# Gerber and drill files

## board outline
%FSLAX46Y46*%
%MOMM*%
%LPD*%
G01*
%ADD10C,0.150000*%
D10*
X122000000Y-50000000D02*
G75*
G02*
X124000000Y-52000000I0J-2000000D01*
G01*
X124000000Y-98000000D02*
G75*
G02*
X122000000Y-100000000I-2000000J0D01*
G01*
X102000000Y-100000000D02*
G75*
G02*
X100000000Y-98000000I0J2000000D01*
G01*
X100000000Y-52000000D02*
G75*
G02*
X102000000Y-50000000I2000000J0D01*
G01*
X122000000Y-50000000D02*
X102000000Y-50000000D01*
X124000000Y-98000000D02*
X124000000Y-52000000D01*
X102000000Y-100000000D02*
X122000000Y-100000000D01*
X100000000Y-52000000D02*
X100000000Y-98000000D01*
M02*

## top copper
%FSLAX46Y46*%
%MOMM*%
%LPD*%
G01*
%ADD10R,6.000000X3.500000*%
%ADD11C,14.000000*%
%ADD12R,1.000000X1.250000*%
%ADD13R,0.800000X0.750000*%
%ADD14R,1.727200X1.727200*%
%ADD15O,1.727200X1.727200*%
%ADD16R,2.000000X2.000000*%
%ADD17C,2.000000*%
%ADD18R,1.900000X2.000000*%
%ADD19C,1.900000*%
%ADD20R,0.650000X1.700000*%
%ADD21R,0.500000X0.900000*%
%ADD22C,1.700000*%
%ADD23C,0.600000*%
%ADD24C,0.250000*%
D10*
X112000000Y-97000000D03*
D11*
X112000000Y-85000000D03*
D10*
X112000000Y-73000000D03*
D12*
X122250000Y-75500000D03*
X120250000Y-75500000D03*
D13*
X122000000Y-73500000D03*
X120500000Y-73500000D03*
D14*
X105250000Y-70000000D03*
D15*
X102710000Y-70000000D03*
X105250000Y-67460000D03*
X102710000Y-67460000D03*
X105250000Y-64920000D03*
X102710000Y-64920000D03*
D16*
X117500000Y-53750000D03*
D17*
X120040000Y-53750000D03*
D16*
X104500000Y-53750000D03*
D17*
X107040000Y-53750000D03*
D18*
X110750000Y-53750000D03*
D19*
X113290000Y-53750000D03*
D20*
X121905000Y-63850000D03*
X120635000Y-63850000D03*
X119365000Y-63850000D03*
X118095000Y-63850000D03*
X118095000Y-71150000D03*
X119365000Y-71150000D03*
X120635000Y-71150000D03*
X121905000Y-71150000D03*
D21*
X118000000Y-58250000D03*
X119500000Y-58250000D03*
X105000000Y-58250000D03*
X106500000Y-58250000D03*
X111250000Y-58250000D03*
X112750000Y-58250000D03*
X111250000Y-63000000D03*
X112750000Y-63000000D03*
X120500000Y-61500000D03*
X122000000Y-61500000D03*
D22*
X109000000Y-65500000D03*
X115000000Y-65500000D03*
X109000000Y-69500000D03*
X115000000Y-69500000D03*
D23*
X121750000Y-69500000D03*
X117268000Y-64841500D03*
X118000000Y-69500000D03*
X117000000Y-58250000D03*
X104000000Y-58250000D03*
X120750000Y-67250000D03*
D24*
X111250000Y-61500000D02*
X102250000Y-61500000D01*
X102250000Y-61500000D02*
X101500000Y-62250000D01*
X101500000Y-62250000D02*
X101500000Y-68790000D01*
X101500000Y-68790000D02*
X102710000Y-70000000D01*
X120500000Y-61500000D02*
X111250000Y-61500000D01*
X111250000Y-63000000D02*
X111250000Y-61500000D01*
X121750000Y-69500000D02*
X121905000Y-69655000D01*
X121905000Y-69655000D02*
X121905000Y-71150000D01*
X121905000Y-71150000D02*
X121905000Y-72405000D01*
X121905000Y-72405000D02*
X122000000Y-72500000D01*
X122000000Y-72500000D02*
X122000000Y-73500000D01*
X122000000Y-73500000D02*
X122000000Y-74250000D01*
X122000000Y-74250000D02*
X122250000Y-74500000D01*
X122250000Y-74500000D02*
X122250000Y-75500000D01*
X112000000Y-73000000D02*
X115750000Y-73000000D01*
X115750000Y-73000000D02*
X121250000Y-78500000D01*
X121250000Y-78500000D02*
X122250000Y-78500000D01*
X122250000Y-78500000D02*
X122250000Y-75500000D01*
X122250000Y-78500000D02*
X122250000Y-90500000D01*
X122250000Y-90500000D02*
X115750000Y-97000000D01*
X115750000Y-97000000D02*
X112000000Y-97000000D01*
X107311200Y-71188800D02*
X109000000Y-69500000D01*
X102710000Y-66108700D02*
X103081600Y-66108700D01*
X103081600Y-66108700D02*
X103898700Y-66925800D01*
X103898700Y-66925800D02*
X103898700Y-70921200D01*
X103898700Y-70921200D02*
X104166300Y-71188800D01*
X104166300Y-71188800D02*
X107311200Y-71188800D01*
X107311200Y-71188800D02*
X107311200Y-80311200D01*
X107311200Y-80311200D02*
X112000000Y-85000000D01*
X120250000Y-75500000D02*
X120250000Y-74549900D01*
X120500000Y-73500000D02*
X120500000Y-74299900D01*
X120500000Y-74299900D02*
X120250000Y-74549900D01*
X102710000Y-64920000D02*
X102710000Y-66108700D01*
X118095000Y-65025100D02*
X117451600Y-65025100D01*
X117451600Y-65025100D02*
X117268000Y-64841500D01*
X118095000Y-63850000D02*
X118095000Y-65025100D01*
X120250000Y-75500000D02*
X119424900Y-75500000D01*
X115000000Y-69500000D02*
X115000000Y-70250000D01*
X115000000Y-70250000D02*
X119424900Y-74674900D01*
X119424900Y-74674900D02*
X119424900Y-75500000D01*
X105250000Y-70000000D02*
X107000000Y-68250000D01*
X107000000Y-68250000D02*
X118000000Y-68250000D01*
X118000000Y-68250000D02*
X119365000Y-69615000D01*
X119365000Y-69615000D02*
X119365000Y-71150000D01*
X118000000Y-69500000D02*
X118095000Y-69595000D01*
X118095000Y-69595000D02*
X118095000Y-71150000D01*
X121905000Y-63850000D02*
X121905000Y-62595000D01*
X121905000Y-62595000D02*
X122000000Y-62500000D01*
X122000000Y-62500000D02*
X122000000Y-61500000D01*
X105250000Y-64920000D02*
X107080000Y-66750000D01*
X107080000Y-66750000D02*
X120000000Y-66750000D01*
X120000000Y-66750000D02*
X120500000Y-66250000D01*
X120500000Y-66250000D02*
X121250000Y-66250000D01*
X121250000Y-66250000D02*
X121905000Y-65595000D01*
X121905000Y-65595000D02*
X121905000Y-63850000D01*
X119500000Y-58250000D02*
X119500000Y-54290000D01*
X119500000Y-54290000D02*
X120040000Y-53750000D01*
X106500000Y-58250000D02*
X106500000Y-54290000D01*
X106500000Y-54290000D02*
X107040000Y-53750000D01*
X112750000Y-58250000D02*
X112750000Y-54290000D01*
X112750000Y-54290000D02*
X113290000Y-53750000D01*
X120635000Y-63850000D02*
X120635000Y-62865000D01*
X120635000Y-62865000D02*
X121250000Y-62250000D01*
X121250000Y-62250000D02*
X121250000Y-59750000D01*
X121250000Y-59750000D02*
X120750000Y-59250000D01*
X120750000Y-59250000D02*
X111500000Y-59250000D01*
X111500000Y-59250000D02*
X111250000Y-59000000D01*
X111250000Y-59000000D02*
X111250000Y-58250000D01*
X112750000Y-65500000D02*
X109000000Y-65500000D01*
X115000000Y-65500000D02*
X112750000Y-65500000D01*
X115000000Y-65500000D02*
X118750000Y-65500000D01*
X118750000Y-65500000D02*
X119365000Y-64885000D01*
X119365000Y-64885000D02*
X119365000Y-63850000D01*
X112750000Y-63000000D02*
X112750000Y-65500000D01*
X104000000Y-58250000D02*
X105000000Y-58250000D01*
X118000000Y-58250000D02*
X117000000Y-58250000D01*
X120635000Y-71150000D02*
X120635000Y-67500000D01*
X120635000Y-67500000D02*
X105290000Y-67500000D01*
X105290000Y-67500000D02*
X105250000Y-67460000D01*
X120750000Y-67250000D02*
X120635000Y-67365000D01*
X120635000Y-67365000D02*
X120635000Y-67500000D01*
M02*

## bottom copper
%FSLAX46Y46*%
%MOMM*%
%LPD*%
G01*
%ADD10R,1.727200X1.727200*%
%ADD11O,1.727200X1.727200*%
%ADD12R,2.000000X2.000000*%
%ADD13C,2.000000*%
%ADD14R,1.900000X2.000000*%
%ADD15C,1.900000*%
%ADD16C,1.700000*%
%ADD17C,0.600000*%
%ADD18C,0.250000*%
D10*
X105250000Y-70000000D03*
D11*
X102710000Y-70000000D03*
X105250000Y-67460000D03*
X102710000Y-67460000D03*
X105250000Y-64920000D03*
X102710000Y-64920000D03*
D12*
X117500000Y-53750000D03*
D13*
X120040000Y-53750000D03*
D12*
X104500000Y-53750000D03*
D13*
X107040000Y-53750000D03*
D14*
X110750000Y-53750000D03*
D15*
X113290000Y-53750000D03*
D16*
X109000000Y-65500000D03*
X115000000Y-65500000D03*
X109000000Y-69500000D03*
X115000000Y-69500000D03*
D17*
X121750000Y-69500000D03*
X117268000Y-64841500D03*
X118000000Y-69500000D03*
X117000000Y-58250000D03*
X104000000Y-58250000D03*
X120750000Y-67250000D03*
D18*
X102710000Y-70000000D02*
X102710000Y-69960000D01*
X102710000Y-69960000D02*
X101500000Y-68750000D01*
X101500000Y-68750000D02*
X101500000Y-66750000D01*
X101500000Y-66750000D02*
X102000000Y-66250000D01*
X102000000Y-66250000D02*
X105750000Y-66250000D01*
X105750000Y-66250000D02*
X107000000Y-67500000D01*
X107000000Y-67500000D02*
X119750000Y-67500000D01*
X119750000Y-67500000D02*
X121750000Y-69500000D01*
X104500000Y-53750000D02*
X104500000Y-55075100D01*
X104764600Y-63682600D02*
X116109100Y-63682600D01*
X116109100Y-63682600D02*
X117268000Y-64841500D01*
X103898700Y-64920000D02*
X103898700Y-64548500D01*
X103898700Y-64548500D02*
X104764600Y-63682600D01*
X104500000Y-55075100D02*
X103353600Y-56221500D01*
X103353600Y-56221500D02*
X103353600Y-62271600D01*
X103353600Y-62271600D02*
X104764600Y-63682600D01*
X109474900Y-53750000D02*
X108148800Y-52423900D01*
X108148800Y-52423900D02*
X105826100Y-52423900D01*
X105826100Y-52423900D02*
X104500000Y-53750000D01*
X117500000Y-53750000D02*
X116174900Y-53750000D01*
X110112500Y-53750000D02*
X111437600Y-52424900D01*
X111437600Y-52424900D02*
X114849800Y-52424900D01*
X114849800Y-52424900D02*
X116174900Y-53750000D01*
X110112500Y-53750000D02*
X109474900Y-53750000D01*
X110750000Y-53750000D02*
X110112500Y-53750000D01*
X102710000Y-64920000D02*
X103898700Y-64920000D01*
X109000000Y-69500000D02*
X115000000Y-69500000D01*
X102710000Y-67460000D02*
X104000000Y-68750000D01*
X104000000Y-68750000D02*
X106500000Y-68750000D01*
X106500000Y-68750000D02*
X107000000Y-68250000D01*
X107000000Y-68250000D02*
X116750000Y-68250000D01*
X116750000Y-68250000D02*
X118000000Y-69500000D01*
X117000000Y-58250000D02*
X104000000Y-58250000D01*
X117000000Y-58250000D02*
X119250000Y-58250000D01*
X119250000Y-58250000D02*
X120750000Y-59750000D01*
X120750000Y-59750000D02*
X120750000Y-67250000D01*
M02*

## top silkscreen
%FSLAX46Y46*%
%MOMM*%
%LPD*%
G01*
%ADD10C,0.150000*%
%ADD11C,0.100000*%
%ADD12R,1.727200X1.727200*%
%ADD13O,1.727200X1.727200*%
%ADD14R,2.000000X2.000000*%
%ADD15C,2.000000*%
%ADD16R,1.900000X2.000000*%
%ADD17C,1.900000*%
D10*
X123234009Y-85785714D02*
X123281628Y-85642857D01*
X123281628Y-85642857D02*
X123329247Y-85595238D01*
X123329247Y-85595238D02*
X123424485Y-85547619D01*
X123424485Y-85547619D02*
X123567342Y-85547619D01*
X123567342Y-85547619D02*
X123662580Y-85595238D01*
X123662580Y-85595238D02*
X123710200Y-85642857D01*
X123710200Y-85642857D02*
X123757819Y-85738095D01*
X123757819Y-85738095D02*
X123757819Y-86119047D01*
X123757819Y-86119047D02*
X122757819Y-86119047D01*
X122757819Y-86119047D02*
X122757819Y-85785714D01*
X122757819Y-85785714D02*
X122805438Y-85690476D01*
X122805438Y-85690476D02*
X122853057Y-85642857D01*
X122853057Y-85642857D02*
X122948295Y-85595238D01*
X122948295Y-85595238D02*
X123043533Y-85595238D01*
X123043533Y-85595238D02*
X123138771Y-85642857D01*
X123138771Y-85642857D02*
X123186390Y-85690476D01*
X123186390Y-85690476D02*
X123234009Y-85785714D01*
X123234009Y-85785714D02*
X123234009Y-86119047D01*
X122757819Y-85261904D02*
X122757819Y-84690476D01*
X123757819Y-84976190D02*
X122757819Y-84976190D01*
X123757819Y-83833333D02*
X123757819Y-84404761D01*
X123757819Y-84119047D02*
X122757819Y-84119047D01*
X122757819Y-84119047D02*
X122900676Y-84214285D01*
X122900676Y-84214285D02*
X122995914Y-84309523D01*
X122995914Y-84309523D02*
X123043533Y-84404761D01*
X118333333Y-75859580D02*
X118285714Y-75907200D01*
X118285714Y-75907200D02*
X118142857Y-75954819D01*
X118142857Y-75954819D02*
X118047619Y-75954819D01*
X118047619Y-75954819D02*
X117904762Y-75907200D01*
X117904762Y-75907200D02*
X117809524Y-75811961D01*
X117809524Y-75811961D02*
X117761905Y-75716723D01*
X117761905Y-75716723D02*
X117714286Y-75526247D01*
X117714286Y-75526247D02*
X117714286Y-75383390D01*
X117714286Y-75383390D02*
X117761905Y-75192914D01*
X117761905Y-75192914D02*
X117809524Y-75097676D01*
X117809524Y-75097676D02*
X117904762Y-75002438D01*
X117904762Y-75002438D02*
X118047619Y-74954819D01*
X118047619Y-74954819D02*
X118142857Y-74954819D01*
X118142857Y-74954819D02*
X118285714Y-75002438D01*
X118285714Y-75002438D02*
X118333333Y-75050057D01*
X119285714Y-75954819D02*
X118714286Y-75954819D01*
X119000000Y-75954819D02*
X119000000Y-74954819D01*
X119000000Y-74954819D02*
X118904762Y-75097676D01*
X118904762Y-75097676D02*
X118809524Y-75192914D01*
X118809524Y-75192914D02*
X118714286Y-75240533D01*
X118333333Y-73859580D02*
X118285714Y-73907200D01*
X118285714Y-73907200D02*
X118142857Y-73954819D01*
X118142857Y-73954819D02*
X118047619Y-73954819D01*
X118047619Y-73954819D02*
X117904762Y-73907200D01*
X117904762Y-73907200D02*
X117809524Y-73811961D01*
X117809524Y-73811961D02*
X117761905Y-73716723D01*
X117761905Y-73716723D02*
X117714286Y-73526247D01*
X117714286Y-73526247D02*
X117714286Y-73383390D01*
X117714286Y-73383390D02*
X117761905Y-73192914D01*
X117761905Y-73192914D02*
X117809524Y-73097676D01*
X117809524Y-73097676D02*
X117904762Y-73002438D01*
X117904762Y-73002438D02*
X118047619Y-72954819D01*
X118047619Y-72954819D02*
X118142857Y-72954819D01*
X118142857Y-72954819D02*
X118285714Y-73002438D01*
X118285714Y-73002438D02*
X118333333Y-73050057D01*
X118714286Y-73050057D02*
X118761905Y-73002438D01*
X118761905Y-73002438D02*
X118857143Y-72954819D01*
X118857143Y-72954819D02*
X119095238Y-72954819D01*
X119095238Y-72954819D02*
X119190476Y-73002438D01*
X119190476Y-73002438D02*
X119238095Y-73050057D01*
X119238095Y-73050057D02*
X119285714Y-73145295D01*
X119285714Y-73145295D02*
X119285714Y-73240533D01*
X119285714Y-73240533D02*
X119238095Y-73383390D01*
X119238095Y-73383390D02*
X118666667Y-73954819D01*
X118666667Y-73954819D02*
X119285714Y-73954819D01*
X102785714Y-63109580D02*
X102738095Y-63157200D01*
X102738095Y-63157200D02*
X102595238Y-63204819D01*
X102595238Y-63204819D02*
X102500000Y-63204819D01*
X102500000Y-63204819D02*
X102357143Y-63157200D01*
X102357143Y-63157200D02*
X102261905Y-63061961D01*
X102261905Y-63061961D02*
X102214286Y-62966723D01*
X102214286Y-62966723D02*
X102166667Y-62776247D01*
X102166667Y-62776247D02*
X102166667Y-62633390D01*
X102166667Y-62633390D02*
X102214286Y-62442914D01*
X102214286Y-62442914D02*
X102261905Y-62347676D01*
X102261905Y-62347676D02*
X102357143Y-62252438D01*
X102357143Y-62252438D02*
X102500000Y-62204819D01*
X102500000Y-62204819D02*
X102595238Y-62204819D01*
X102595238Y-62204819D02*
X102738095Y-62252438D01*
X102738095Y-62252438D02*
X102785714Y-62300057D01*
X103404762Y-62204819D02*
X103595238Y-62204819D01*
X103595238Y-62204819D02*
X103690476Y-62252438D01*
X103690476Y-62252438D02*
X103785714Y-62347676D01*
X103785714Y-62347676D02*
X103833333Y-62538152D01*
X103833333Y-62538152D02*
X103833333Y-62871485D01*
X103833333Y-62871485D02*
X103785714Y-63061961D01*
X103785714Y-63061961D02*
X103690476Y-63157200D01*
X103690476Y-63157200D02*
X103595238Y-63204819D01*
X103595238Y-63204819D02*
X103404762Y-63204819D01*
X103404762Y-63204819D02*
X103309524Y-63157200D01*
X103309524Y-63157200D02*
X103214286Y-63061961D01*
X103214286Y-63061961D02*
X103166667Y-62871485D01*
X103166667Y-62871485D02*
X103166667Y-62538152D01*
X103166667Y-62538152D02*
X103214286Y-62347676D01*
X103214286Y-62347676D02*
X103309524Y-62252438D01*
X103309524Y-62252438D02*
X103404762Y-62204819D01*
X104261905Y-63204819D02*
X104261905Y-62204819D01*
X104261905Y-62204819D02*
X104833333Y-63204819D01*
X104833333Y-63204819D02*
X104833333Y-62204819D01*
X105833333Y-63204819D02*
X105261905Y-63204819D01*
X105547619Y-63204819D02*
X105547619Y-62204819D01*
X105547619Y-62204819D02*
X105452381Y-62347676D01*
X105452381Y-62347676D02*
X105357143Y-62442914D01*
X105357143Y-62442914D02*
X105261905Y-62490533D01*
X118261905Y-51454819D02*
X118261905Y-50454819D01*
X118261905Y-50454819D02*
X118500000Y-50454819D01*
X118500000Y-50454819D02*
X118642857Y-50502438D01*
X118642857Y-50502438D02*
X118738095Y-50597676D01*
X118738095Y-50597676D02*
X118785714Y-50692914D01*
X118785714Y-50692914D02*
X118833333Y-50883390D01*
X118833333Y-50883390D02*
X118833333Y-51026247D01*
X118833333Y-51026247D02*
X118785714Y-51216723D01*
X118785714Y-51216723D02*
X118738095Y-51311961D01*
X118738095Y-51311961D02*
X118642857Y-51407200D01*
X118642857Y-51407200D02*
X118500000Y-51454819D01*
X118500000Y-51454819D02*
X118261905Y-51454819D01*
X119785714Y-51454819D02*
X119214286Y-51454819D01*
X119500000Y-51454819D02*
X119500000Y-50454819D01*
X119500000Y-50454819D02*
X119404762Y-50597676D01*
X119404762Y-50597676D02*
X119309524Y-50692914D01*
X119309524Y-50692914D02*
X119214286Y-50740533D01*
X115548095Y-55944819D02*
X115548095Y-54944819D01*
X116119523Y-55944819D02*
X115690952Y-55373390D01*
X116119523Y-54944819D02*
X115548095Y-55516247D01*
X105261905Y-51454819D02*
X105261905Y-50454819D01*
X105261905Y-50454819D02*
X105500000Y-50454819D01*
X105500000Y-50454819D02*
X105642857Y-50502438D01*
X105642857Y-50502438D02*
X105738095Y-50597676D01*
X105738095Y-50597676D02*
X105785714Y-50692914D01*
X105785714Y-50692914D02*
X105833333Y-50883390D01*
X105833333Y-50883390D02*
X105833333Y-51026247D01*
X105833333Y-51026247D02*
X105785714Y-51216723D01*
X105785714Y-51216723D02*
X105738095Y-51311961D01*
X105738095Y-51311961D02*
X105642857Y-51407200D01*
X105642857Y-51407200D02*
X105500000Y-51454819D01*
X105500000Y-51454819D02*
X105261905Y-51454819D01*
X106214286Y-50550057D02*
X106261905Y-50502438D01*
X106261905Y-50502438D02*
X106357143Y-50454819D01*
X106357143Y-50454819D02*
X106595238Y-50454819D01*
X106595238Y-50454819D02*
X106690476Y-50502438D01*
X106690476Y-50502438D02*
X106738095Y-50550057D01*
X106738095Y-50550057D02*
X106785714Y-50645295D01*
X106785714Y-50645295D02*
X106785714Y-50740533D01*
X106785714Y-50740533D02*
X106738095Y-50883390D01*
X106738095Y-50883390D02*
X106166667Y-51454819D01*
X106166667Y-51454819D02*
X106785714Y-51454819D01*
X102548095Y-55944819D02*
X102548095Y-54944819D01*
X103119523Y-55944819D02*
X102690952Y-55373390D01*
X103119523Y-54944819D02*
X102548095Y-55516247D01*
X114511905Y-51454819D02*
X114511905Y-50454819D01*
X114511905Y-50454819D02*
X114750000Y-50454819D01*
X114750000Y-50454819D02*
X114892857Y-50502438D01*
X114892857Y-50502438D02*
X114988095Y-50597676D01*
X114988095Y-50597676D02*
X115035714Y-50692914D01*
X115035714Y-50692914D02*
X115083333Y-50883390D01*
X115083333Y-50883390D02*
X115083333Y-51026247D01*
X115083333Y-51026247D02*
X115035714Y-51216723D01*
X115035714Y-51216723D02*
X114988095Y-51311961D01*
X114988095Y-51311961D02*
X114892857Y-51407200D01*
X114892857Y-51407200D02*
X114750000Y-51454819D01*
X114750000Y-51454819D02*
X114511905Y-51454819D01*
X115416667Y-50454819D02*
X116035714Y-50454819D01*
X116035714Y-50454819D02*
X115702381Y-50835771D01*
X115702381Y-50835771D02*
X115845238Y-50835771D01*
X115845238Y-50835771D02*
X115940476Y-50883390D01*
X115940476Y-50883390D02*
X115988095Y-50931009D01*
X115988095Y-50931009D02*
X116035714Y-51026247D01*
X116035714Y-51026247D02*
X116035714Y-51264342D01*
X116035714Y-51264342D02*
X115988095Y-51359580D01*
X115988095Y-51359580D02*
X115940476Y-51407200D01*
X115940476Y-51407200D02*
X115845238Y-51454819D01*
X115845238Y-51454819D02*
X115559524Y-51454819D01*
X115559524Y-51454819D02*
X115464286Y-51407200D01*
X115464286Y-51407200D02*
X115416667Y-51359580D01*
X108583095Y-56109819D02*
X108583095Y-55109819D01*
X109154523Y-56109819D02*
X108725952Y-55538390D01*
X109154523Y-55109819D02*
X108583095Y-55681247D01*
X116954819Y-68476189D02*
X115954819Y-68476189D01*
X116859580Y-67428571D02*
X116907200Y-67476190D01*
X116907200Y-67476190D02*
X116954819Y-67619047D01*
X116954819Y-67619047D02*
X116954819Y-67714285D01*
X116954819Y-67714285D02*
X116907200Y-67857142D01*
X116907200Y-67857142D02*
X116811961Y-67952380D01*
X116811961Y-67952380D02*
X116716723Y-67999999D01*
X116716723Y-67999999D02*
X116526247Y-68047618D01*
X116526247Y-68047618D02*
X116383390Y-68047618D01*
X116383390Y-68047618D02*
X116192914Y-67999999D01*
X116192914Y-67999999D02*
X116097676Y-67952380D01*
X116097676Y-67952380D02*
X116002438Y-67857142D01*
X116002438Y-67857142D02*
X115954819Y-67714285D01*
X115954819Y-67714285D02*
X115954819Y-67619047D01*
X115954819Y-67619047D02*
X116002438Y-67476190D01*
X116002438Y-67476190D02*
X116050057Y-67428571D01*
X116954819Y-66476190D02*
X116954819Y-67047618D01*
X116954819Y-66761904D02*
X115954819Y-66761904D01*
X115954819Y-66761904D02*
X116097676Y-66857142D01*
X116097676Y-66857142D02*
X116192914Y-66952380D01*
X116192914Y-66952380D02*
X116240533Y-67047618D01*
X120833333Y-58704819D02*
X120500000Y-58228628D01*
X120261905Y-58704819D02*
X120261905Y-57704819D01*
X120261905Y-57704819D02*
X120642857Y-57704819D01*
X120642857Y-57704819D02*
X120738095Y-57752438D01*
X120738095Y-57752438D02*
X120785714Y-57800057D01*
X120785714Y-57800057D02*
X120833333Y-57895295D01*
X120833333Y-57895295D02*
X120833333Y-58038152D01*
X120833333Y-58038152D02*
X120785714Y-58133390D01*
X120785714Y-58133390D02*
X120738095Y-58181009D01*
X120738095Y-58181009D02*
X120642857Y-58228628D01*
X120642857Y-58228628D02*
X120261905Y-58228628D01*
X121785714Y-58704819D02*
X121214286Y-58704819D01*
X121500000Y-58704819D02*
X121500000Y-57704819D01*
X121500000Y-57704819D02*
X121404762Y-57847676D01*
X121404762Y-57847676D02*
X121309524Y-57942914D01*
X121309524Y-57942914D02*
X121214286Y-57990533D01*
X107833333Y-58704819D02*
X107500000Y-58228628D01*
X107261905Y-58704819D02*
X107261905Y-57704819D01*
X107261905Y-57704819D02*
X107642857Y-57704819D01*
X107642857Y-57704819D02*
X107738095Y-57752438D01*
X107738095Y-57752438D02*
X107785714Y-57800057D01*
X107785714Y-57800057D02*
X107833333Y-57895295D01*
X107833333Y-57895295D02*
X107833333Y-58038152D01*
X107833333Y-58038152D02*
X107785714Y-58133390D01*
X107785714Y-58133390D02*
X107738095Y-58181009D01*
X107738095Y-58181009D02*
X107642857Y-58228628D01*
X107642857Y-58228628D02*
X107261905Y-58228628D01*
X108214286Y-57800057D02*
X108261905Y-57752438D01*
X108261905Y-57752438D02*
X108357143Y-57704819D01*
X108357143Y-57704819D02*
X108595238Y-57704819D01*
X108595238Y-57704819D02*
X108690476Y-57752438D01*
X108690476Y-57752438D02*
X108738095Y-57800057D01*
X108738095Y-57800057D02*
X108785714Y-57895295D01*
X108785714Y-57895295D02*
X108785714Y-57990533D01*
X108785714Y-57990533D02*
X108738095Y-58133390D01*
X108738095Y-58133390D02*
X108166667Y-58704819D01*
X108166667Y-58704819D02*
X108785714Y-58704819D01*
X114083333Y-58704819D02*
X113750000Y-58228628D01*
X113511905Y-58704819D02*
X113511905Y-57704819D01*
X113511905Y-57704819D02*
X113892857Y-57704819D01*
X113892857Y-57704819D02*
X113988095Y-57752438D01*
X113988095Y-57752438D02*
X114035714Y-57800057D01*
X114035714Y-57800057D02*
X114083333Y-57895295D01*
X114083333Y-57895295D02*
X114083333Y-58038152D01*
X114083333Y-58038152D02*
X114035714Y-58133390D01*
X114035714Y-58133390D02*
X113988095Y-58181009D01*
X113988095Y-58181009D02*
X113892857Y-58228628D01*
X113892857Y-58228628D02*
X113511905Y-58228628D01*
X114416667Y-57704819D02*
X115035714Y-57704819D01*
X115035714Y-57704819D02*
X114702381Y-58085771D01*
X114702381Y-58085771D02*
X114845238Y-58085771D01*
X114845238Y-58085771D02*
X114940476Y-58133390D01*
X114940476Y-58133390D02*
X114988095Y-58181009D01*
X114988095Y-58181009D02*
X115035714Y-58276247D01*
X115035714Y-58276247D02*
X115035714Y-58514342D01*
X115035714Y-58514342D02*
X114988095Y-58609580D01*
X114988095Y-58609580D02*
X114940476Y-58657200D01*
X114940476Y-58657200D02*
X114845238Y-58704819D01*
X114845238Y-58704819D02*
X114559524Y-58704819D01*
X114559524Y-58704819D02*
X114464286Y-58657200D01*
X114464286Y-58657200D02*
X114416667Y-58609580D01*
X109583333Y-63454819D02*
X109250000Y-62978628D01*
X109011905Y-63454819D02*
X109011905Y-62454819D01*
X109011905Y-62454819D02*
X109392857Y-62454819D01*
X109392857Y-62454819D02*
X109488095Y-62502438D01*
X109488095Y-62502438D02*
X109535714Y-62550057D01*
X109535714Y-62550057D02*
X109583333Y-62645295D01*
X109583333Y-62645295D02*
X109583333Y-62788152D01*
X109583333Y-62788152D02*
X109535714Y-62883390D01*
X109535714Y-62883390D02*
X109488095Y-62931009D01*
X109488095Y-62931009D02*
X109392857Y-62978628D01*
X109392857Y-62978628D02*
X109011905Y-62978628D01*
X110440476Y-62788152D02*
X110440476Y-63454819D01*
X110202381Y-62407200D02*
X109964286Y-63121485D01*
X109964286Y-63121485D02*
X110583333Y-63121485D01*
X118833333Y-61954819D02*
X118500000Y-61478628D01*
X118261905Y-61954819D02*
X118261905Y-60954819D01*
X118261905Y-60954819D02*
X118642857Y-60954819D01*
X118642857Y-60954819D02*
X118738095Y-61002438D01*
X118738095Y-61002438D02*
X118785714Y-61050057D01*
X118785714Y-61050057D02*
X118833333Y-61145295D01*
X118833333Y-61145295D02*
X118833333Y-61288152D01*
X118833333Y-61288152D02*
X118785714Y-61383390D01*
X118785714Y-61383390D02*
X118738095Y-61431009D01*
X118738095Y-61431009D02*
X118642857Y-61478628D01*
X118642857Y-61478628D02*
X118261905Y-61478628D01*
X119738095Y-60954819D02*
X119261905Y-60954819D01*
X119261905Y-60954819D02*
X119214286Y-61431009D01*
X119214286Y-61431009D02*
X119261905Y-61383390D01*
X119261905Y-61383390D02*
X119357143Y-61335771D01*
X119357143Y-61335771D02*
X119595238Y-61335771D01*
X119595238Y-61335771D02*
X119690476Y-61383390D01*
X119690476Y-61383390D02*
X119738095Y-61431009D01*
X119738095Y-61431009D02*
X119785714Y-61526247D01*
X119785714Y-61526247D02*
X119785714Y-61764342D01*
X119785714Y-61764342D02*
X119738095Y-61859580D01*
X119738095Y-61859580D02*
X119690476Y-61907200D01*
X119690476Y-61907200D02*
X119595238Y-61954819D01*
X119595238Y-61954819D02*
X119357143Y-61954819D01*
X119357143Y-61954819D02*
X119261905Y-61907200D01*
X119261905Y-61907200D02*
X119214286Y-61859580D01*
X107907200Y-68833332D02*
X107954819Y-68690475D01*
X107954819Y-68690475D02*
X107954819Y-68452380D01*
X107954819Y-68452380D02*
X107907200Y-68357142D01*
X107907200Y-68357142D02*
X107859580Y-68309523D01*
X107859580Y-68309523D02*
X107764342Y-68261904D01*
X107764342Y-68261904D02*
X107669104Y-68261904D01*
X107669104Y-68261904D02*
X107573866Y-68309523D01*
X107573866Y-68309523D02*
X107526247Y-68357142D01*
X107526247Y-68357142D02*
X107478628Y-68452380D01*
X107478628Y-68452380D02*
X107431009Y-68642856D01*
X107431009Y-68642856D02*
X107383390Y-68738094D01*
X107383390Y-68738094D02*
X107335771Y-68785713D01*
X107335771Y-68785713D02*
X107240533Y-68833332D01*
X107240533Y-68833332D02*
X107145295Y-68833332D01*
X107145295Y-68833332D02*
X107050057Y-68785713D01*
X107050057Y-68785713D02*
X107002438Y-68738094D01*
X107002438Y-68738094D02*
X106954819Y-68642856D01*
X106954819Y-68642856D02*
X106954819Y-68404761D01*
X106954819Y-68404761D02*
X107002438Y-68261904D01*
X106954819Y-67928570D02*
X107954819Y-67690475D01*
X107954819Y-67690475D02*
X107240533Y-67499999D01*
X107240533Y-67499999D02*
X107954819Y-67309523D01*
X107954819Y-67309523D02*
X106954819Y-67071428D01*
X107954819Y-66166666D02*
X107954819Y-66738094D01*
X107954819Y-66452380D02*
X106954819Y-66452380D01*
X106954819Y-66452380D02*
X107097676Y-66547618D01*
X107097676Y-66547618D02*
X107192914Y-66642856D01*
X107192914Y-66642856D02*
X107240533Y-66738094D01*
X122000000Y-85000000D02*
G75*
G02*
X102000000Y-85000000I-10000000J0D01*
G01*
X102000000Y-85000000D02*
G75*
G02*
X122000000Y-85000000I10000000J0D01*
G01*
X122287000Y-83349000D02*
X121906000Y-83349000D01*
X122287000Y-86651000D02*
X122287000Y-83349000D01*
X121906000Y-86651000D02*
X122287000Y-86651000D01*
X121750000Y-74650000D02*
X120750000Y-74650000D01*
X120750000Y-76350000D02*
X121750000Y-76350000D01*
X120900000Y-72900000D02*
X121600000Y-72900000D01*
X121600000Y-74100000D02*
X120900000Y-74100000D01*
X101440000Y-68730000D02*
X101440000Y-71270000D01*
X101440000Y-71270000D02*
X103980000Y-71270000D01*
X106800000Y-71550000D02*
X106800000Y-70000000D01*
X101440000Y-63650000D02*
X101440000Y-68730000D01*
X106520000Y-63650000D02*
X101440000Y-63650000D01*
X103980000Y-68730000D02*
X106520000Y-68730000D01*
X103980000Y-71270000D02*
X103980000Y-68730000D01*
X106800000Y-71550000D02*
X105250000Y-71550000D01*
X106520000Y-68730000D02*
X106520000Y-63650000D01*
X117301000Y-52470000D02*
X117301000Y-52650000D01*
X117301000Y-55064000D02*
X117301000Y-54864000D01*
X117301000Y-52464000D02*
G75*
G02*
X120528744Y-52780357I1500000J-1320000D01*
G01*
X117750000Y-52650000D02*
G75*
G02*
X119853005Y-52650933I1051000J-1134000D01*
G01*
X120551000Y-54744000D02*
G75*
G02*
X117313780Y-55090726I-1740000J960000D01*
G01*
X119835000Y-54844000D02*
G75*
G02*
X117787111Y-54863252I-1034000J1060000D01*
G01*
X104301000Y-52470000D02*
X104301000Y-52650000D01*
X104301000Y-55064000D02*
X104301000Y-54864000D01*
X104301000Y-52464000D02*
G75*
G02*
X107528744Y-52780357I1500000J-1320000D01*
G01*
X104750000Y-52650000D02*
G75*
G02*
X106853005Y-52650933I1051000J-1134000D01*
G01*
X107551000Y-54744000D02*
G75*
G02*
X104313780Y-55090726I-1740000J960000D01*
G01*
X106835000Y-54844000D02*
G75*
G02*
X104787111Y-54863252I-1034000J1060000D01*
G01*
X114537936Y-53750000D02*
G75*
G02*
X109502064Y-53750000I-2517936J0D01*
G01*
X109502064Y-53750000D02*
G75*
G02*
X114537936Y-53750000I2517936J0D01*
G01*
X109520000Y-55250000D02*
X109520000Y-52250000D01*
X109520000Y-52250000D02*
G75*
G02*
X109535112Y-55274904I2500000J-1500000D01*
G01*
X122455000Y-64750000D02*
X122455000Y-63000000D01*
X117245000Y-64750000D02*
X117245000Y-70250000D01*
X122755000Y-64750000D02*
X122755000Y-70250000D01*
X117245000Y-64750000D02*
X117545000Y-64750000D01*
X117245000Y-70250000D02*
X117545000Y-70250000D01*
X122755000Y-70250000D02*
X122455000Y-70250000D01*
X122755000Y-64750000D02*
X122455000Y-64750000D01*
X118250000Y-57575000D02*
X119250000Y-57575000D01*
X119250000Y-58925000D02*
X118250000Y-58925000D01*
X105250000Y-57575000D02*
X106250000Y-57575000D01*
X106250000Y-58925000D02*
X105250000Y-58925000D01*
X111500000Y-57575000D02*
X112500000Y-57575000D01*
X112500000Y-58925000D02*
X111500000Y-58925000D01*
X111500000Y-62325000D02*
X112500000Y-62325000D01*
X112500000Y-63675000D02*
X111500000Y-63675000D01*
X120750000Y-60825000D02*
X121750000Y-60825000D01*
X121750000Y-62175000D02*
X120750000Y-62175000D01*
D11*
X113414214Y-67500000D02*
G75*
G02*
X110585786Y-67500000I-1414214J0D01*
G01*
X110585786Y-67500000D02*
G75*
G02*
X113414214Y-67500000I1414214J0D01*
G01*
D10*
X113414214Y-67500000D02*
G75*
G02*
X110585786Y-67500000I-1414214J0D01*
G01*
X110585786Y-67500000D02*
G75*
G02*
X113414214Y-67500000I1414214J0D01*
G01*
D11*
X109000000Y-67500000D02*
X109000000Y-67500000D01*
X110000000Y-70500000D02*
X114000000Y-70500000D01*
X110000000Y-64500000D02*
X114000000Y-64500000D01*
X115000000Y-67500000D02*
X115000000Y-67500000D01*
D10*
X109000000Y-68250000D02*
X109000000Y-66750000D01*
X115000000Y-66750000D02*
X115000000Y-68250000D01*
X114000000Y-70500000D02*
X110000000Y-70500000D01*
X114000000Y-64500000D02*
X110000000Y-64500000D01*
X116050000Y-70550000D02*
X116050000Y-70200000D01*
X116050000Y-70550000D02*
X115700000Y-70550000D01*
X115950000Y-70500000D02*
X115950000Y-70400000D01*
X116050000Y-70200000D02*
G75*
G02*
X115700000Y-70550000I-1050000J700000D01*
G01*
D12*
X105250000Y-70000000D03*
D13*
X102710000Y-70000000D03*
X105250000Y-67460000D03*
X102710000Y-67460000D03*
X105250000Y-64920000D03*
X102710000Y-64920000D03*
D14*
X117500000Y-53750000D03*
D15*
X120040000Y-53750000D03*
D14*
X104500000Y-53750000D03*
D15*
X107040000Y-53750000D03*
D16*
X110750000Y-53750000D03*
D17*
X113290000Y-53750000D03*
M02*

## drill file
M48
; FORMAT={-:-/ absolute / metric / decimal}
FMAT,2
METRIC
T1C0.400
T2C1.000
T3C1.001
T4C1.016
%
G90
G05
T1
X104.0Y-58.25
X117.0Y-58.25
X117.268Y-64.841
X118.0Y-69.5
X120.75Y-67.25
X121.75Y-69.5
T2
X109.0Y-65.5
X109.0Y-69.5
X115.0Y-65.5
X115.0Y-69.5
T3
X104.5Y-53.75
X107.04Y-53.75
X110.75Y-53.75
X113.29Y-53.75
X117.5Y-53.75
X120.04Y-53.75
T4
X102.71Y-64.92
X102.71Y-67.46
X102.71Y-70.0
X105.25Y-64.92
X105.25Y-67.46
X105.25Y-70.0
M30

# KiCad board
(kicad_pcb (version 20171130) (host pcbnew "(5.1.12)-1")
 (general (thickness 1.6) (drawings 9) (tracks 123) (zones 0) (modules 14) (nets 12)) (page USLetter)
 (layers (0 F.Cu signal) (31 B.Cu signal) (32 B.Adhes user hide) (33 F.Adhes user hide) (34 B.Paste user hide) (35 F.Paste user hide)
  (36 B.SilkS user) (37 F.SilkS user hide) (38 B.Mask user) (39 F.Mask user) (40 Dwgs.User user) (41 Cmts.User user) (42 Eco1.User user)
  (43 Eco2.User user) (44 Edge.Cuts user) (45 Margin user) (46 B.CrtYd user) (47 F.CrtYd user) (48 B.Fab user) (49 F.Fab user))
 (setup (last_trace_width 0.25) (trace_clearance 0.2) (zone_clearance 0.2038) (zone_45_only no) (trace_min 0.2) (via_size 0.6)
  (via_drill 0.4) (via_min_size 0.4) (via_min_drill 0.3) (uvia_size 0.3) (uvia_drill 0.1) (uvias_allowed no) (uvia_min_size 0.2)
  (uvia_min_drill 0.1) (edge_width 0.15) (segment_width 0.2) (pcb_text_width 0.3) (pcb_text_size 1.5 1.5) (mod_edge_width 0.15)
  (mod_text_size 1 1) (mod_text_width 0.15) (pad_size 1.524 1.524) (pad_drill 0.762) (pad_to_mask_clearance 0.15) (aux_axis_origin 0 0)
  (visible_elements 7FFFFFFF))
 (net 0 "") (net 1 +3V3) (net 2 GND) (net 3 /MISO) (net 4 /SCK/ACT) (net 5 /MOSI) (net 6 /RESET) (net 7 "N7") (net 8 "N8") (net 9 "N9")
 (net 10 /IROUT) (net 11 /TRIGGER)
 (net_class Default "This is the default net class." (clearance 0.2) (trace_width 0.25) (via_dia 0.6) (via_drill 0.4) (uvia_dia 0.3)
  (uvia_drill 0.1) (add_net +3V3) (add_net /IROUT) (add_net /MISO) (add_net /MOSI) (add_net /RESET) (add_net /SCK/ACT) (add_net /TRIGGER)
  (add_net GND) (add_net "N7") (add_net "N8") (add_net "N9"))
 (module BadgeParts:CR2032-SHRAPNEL (layer F.Cu) (at 112 85 90)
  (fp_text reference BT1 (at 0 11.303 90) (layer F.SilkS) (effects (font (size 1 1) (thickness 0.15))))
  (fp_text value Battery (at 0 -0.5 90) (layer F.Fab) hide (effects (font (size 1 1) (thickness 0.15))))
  (fp_circle (center 0 0) (end 10 0) (layer F.SilkS) (width 0.15))
  (fp_line (start 1.651 10.287) (end 1.651 9.906) (layer F.SilkS) (width 0.15))
  (fp_line (start -1.651 10.287) (end 1.651 10.287) (layer F.SilkS) (width 0.15))
  (fp_line (start -1.651 9.906) (end -1.651 10.287) (layer F.SilkS) (width 0.15))
  (pad 1 smd rect (at -12 0 90) (size 3.5 6) (layers F.Cu F.Paste F.Mask) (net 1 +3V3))
  (pad 2 smd circle (at 0 0 90) (size 14 14) (layers F.Cu F.Paste F.Mask) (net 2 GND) (solder_mask_margin 3) (thermal_gap 3))
  (pad 1 smd rect (at 12 0 90) (size 3.5 6) (layers F.Cu F.Paste F.Mask) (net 1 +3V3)))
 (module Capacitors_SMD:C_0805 (layer F.Cu) (at 121.25 75.5 180)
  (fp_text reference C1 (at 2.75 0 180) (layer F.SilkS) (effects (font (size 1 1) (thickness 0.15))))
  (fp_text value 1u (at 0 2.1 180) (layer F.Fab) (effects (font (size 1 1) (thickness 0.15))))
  (fp_line (start -0.5 0.85) (end 0.5 0.85) (layer F.SilkS) (width 0.15))
  (fp_line (start 0.5 -0.85) (end -0.5 -0.85) (layer F.SilkS) (width 0.15))
  (pad 1 smd rect (at -1 0 180) (size 1 1.25) (layers F.Cu F.Paste F.Mask) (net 1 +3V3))
  (pad 2 smd rect (at 1 0 180) (size 1 1.25) (layers F.Cu F.Paste F.Mask) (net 2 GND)))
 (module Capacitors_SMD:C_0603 (layer F.Cu) (at 121.25 73.5 180)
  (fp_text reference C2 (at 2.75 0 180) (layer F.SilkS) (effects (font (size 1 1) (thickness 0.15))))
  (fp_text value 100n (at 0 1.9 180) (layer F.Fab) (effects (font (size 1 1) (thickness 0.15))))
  (fp_line (start 0.35 0.6) (end -0.35 0.6) (layer F.SilkS) (width 0.15))
  (fp_line (start -0.35 -0.6) (end 0.35 -0.6) (layer F.SilkS) (width 0.15))
  (pad 1 smd rect (at -0.75 0 180) (size 0.8 0.75) (layers F.Cu F.Paste F.Mask) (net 1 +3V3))
  (pad 2 smd rect (at 0.75 0 180) (size 0.8 0.75) (layers F.Cu F.Paste F.Mask) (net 2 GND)))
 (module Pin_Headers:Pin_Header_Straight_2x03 (layer F.Cu) (at 105.25 70 180)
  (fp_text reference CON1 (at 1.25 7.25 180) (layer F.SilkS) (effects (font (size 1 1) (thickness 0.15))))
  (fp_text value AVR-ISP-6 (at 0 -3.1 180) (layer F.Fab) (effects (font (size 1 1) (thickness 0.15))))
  (fp_line (start 3.81 1.27) (end 3.81 -1.27) (layer F.SilkS) (width 0.15))
  (fp_line (start 3.81 -1.27) (end 1.27 -1.27) (layer F.SilkS) (width 0.15))
  (fp_line (start -1.55 -1.55) (end -1.55 0) (layer F.SilkS) (width 0.15))
  (fp_line (start 3.81 6.35) (end 3.81 1.27) (layer F.SilkS) (width 0.15))
  (fp_line (start -1.27 6.35) (end 3.81 6.35) (layer F.SilkS) (width 0.15))
  (fp_line (start 1.27 1.27) (end -1.27 1.27) (layer F.SilkS) (width 0.15))
  (fp_line (start 1.27 -1.27) (end 1.27 1.27) (layer F.SilkS) (width 0.15))
  (fp_line (start -1.55 -1.55) (end 0 -1.55) (layer F.SilkS) (width 0.15))
  (fp_line (start -1.27 1.27) (end -1.27 6.35) (layer F.SilkS) (width 0.15))
  (pad 1 thru_hole rect (at 0 0 180) (size 1.7272 1.7272) (drill 1.016) (layers *.Cu *.Mask F.SilkS) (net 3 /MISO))
  (pad 2 thru_hole oval (at 2.54 0 180) (size 1.7272 1.7272) (drill 1.016) (layers *.Cu *.Mask F.SilkS) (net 1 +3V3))
  (pad 3 thru_hole oval (at 0 2.54 180) (size 1.7272 1.7272) (drill 1.016) (layers *.Cu *.Mask F.SilkS) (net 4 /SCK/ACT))
  (pad 4 thru_hole oval (at 2.54 2.54 180) (size 1.7272 1.7272) (drill 1.016) (layers *.Cu *.Mask F.SilkS) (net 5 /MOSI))
  (pad 5 thru_hole oval (at 0 5.08 180) (size 1.7272 1.7272) (drill 1.016) (layers *.Cu *.Mask F.SilkS) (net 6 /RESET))
  (pad 6 thru_hole oval (at 2.54 5.08 180) (size 1.7272 1.7272) (drill 1.016) (layers *.Cu *.Mask F.SilkS) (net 2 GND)))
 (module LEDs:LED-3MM (layer F.Cu) (at 117.5 53.75)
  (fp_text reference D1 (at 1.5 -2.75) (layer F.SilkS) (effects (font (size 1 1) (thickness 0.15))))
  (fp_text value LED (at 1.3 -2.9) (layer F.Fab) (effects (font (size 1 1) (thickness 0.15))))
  (fp_line (start -0.199 -1.28) (end -0.199 -1.1) (layer F.SilkS) (width 0.15))
  (fp_line (start -0.199 1.314) (end -0.199 1.114) (layer F.SilkS) (width 0.15))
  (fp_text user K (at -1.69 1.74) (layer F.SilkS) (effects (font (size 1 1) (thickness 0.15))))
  (fp_arc (start 1.301 0.034) (end -0.199 -1.286) (angle 108.5) (layer F.SilkS) (width 0.15))
  (fp_arc (start 1.301 0.034) (end 0.25 -1.1) (angle 85.7) (layer F.SilkS) (width 0.15))
  (fp_arc (start 1.311 0.034) (end 3.051 0.994) (angle 110) (layer F.SilkS) (width 0.15))
  (fp_arc (start 1.301 0.034) (end 2.335 1.094) (angle 87.5) (layer F.SilkS) (width 0.15))
  (pad 1 thru_hole rect (at 0 0 90) (size 2 2) (drill 1.00076) (layers *.Cu *.Mask F.SilkS) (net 2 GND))
  (pad 2 thru_hole circle (at 2.54 0) (size 2 2) (drill 1.00076) (layers *.Cu *.Mask F.SilkS) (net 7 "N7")))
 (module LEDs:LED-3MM (layer F.Cu) (at 104.5 53.75)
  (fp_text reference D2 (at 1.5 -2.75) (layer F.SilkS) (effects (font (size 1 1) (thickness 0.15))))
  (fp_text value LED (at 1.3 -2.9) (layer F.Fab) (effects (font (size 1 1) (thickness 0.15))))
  (fp_line (start -0.199 -1.28) (end -0.199 -1.1) (layer F.SilkS) (width 0.15))
  (fp_line (start -0.199 1.314) (end -0.199 1.114) (layer F.SilkS) (width 0.15))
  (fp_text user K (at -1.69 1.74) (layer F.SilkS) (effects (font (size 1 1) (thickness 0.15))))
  (fp_arc (start 1.301 0.034) (end -0.199 -1.286) (angle 108.5) (layer F.SilkS) (width 0.15))
  (fp_arc (start 1.301 0.034) (end 0.25 -1.1) (angle 85.7) (layer F.SilkS) (width 0.15))
  (fp_arc (start 1.311 0.034) (end 3.051 0.994) (angle 110) (layer F.SilkS) (width 0.15))
  (fp_arc (start 1.301 0.034) (end 2.335 1.094) (angle 87.5) (layer F.SilkS) (width 0.15))
  (pad 1 thru_hole rect (at 0 0 90) (size 2 2) (drill 1.00076) (layers *.Cu *.Mask F.SilkS) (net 2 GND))
  (pad 2 thru_hole circle (at 2.54 0) (size 2 2) (drill 1.00076) (layers *.Cu *.Mask F.SilkS) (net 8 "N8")))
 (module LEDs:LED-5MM (layer F.Cu) (at 110.75 53.75)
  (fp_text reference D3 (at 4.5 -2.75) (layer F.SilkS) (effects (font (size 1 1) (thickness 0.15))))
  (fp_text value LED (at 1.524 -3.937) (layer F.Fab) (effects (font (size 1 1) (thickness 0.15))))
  (fp_circle (center 1.27 0) (end 0.97 -2.5) (layer F.SilkS) (width 0.15))
  (fp_line (start -1.23 1.5) (end -1.23 -1.5) (layer F.SilkS) (width 0.15))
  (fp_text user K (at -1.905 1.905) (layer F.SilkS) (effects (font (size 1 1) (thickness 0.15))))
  (fp_arc (start 1.27 0) (end -1.23 -1.5) (angle 297.5) (layer F.SilkS) (width 0.15))
  (pad 1 thru_hole rect (at 0 0 90) (size 2 1.9) (drill 1.00076) (layers *.Cu *.Mask F.SilkS) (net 2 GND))
  (pad 2 thru_hole circle (at 2.54 0) (size 1.9 1.9) (drill 1.00076) (layers *.Cu *.Mask F.SilkS) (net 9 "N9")))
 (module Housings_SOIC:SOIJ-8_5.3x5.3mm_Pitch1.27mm (layer F.Cu) (at 120 67.5 270)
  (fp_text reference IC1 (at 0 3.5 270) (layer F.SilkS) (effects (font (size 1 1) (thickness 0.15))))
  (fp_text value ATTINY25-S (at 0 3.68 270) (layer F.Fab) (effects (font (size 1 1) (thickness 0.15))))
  (fp_line (start -2.75 -2.455) (end -4.5 -2.455) (layer F.SilkS) (width 0.15))
  (fp_line (start -2.75 2.755) (end 2.75 2.755) (layer F.SilkS) (width 0.15))
  (fp_line (start -2.75 -2.755) (end 2.75 -2.755) (layer F.SilkS) (width 0.15))
  (fp_line (start -2.75 2.755) (end -2.75 2.455) (layer F.SilkS) (width 0.15))
  (fp_line (start 2.75 2.755) (end 2.75 2.455) (layer F.SilkS) (width 0.15))
  (fp_line (start 2.75 -2.755) (end 2.75 -2.455) (layer F.SilkS) (width 0.15))
  (fp_line (start -2.75 -2.755) (end -2.75 -2.455) (layer F.SilkS) (width 0.15))
  (pad 1 smd rect (at -3.65 -1.905 270) (size 1.7 0.65) (layers F.Cu F.Paste F.Mask) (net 6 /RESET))
  (pad 2 smd rect (at -3.65 -0.635 270) (size 1.7 0.65) (layers F.Cu F.Paste F.Mask) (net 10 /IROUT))
  (pad 3 smd rect (at -3.65 0.635 270) (size 1.7 0.65) (layers F.Cu F.Paste F.Mask) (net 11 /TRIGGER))
  (pad 4 smd rect (at -3.65 1.905 270) (size 1.7 0.65) (layers F.Cu F.Paste F.Mask) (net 2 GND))
  (pad 5 smd rect (at 3.65 1.905 270) (size 1.7 0.65) (layers F.Cu F.Paste F.Mask) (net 5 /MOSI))
  (pad 6 smd rect (at 3.65 0.635 270) (size 1.7 0.65) (layers F.Cu F.Paste F.Mask) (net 3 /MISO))
  (pad 7 smd rect (at 3.65 -0.635 270) (size 1.7 0.65) (layers F.Cu F.Paste F.Mask) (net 4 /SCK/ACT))
  (pad 8 smd rect (at 3.65 -1.905 270) (size 1.7 0.65) (layers F.Cu F.Paste F.Mask) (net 1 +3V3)))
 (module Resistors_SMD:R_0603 (layer F.Cu) (at 118.75 58.25)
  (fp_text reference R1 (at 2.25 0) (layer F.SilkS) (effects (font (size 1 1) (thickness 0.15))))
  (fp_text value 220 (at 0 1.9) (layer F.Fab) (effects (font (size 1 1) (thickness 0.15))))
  (fp_line (start -0.5 -0.675) (end 0.5 -0.675) (layer F.SilkS) (width 0.15))
  (fp_line (start 0.5 0.675) (end -0.5 0.675) (layer F.SilkS) (width 0.15))
  (pad 1 smd rect (at -0.75 0) (size 0.5 0.9) (layers F.Cu F.Paste F.Mask) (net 4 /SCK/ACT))
  (pad 2 smd rect (at 0.75 0) (size 0.5 0.9) (layers F.Cu F.Paste F.Mask) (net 7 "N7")))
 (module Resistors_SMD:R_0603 (layer F.Cu) (at 105.75 58.25)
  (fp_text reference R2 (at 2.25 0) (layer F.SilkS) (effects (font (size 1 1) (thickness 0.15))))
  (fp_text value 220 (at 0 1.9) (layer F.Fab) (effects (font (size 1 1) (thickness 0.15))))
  (fp_line (start -0.5 -0.675) (end 0.5 -0.675) (layer F.SilkS) (width 0.15))
  (fp_line (start 0.5 0.675) (end -0.5 0.675) (layer F.SilkS) (width 0.15))
  (pad 1 smd rect (at -0.75 0) (size 0.5 0.9) (layers F.Cu F.Paste F.Mask) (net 4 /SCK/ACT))
  (pad 2 smd rect (at 0.75 0) (size 0.5 0.9) (layers F.Cu F.Paste F.Mask) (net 8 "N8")))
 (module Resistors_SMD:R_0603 (layer F.Cu) (at 112 58.25)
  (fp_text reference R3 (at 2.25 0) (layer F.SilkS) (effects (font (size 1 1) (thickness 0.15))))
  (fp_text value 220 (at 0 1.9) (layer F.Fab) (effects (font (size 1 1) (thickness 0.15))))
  (fp_line (start -0.5 -0.675) (end 0.5 -0.675) (layer F.SilkS) (width 0.15))
  (fp_line (start 0.5 0.675) (end -0.5 0.675) (layer F.SilkS) (width 0.15))
  (pad 1 smd rect (at -0.75 0) (size 0.5 0.9) (layers F.Cu F.Paste F.Mask) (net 10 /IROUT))
  (pad 2 smd rect (at 0.75 0) (size 0.5 0.9) (layers F.Cu F.Paste F.Mask) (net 9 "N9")))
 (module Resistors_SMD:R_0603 (layer F.Cu) (at 112 63)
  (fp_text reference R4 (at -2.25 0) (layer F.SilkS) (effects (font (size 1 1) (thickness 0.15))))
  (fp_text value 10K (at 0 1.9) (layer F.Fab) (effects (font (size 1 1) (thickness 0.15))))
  (fp_line (start -0.5 -0.675) (end 0.5 -0.675) (layer F.SilkS) (width 0.15))
  (fp_line (start 0.5 0.675) (end -0.5 0.675) (layer F.SilkS) (width 0.15))
  (pad 1 smd rect (at -0.75 0) (size 0.5 0.9) (layers F.Cu F.Paste F.Mask) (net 1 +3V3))
  (pad 2 smd rect (at 0.75 0) (size 0.5 0.9) (layers F.Cu F.Paste F.Mask) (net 11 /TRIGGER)))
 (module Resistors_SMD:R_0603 (layer F.Cu) (at 121.25 61.5)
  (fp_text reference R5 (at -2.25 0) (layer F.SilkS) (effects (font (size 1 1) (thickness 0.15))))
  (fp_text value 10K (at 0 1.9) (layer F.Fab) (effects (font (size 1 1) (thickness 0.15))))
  (fp_line (start -0.5 -0.675) (end 0.5 -0.675) (layer F.SilkS) (width 0.15))
  (fp_line (start 0.5 0.675) (end -0.5 0.675) (layer F.SilkS) (width 0.15))
  (pad 1 smd rect (at -0.75 0) (size 0.5 0.9) (layers F.Cu F.Paste F.Mask) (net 1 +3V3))
  (pad 2 smd rect (at 0.75 0) (size 0.5 0.9) (layers F.Cu F.Paste F.Mask) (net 6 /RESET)))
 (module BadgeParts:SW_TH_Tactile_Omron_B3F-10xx (layer F.Cu) (at 115 69.5 180)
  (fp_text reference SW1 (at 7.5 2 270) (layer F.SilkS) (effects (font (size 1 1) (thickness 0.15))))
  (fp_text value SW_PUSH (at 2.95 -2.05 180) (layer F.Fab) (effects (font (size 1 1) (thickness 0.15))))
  (fp_circle (center 3 2) (end 4 3) (layer F.SilkS) (width 0.1))
  (fp_circle (center 3 2) (end 4 3) (layer F.SilkS) (width 0.15)) (fp_line (start 6 2) (end 6 2) (layer F.SilkS) (width 0.1))
  (fp_line (start 5 -1) (end 1 -1) (layer F.SilkS) (width 0.1)) (fp_line (start 5 5) (end 1 5) (layer F.SilkS) (width 0.1))
  (fp_line (start 0 2) (end 0 2) (layer F.SilkS) (width 0.1))
  (fp_line (start 6 1.25) (end 6 2.75) (layer F.SilkS) (width 0.15))
  (fp_line (start 0 2.75) (end 0 1.25) (layer F.SilkS) (width 0.15))
  (fp_line (start 1 -1) (end 5 -1) (layer F.SilkS) (width 0.15)) (fp_line (start 1 5) (end 5 5) (layer F.SilkS) (width 0.15))
  (fp_line (start -1.05 -1.05) (end -1.05 -0.7) (layer F.SilkS) (width 0.15))
  (fp_line (start -1.05 -1.05) (end -0.7 -1.05) (layer F.SilkS) (width 0.15))
  (fp_line (start -0.95 -1) (end -0.95 -0.9) (layer F.SilkS) (width 0.15))
  (fp_arc (start 0 0) (end -1.05 -0.7) (angle 22.61986495) (layer F.SilkS) (width 0.15))
  (pad 2 thru_hole circle (at 6 4 180) (size 1.7 1.7) (drill 1) (layers *.Cu *.Mask) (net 11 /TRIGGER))
  (pad 2 thru_hole circle (at 0 4 180) (size 1.7 1.7) (drill 1) (layers *.Cu *.Mask) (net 11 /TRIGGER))
  (pad 1 thru_hole circle (at 6 0 180) (size 1.7 1.7) (drill 1) (layers *.Cu *.Mask) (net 2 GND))
  (pad 1 thru_hole circle (at 0 0 180) (size 1.7 1.7) (drill 1) (layers *.Cu *.Mask) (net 2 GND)))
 (gr_arc (start 122 52) (end 122 50) (angle 90) (layer Edge.Cuts) (width 0.15))
 (gr_arc (start 122 98) (end 124 98) (angle 90) (layer Edge.Cuts) (width 0.15))
 (gr_arc (start 102 98) (end 102 100) (angle 90) (layer Edge.Cuts) (width 0.15))
 (gr_arc (start 102 52) (end 100 52) (angle 90) (layer Edge.Cuts) (width 0.15))
 (gr_line (start 122 50) (end 102 50) (angle 90) (layer Edge.Cuts) (width 0.15))
 (gr_line (start 124 98) (end 124 52) (angle 90) (layer Edge.Cuts) (width 0.15))
 (gr_line (start 102 100) (end 122 100) (angle 90) (layer Edge.Cuts) (width 0.15))
 (gr_line (start 100 52) (end 100 98) (angle 90) (layer Edge.Cuts) (width 0.15))
 (segment (start 111.25 61.5) (end 102.25 61.5) (width 0.25) (layer F.Cu) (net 1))
 (segment (start 102.25 61.5) (end 101.5 62.25) (width 0.25) (layer F.Cu) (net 1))
 (segment (start 101.5 62.25) (end 101.5 68.79) (width 0.25) (layer F.Cu) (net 1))
 (segment (start 101.5 68.79) (end 102.71 70) (width 0.25) (layer F.Cu) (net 1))
 (segment (start 120.5 61.5) (end 111.25 61.5) (width 0.25) (layer F.Cu) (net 1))
 (segment (start 111.25 63) (end 111.25 61.5) (width 0.25) (layer F.Cu) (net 1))
 (segment (start 102.71 70) (end 102.71 69.96) (width 0.25) (layer B.Cu) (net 1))
 (segment (start 102.71 69.96) (end 101.5 68.75) (width 0.25) (layer B.Cu) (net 1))
 (segment (start 101.5 68.75) (end 101.5 66.75) (width 0.25) (layer B.Cu) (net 1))
 (segment (start 101.5 66.75) (end 102 66.25) (width 0.25) (layer B.Cu) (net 1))
 (segment (start 102 66.25) (end 105.75 66.25) (width 0.25) (layer B.Cu) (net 1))
 (segment (start 105.75 66.25) (end 107 67.5) (width 0.25) (layer B.Cu) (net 1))
 (segment (start 107 67.5) (end 119.75 67.5) (width 0.25) (layer B.Cu) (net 1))
 (segment (start 119.75 67.5) (end 121.75 69.5) (width 0.25) (layer B.Cu) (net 1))
 (segment (start 121.75 69.5) (end 121.905 69.655) (width 0.25) (layer F.Cu) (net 1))
 (segment (start 121.905 69.655) (end 121.905 71.15) (width 0.25) (layer F.Cu) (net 1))
 (segment (start 121.905 71.15) (end 121.905 72.405) (width 0.25) (layer F.Cu) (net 1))
 (segment (start 121.905 72.405) (end 122 72.5) (width 0.25) (layer F.Cu) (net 1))
 (segment (start 122 72.5) (end 122 73.5) (width 0.25) (layer F.Cu) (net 1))
 (segment (start 122 73.5) (end 122 74.25) (width 0.25) (layer F.Cu) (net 1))
 (segment (start 122 74.25) (end 122.25 74.5) (width 0.25) (layer F.Cu) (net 1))
 (segment (start 122.25 74.5) (end 122.25 75.5) (width 0.25) (layer F.Cu) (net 1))
 (segment (start 112 73) (end 115.75 73) (width 0.25) (layer F.Cu) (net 1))
 (segment (start 115.75 73) (end 121.25 78.5) (width 0.25) (layer F.Cu) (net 1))
 (segment (start 121.25 78.5) (end 122.25 78.5) (width 0.25) (layer F.Cu) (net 1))
 (segment (start 122.25 78.5) (end 122.25 75.5) (width 0.25) (layer F.Cu) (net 1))
 (segment (start 122.25 78.5) (end 122.25 90.5) (width 0.25) (layer F.Cu) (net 1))
 (segment (start 122.25 90.5) (end 115.75 97) (width 0.25) (layer F.Cu) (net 1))
 (segment (start 115.75 97) (end 112 97) (width 0.25) (layer F.Cu) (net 1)) (via (at 121.75 69.5) (size 0.6) (layers F.Cu B.Cu) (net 1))
 (segment (start 107.3112 71.1888) (end 109 69.5) (width 0.25) (layer F.Cu) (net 2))
 (segment (start 102.71 66.1087) (end 103.0816 66.1087) (width 0.25) (layer F.Cu) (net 2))
 (segment (start 103.0816 66.1087) (end 103.8987 66.9258) (width 0.25) (layer F.Cu) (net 2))
 (segment (start 103.8987 66.9258) (end 103.8987 70.9212) (width 0.25) (layer F.Cu) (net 2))
 (segment (start 103.8987 70.9212) (end 104.1663 71.1888) (width 0.25) (layer F.Cu) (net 2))
 (segment (start 104.1663 71.1888) (end 107.3112 71.1888) (width 0.25) (layer F.Cu) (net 2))
 (segment (start 107.3112 71.1888) (end 107.3112 80.3112) (width 0.25) (layer F.Cu) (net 2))
 (segment (start 107.3112 80.3112) (end 112 85) (width 0.25) (layer F.Cu) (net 2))
 (segment (start 120.25 75.5) (end 120.25 74.5499) (width 0.25) (layer F.Cu) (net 2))
 (segment (start 120.5 73.5) (end 120.5 74.2999) (width 0.25) (layer F.Cu) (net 2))
 (segment (start 120.5 74.2999) (end 120.25 74.5499) (width 0.25) (layer F.Cu) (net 2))
 (segment (start 102.71 64.92) (end 102.71 66.1087) (width 0.25) (layer F.Cu) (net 2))
 (segment (start 104.5 53.75) (end 104.5 55.0751) (width 0.25) (layer B.Cu) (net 2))
 (segment (start 104.7646 63.6826) (end 116.1091 63.6826) (width 0.25) (layer B.Cu) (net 2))
 (segment (start 116.1091 63.6826) (end 117.268 64.8415) (width 0.25) (layer B.Cu) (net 2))
 (segment (start 103.8987 64.92) (end 103.8987 64.5485) (width 0.25) (layer B.Cu) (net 2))
 (segment (start 103.8987 64.5485) (end 104.7646 63.6826) (width 0.25) (layer B.Cu) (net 2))
 (segment (start 104.5 55.0751) (end 103.3536 56.2215) (width 0.25) (layer B.Cu) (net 2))
 (segment (start 103.3536 56.2215) (end 103.3536 62.2716) (width 0.25) (layer B.Cu) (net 2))
 (segment (start 103.3536 62.2716) (end 104.7646 63.6826) (width 0.25) (layer B.Cu) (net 2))
 (segment (start 109.4749 53.75) (end 108.1488 52.4239) (width 0.25) (layer B.Cu) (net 2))
 (segment (start 108.1488 52.4239) (end 105.8261 52.4239) (width 0.25) (layer B.Cu) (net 2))
 (segment (start 105.8261 52.4239) (end 104.5 53.75) (width 0.25) (layer B.Cu) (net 2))
 (segment (start 117.5 53.75) (end 116.1749 53.75) (width 0.25) (layer B.Cu) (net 2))
 (segment (start 110.1125 53.75) (end 111.4376 52.4249) (width 0.25) (layer B.Cu) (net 2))
 (segment (start 111.4376 52.4249) (end 114.8498 52.4249) (width 0.25) (layer B.Cu) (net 2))
 (segment (start 114.8498 52.4249) (end 116.1749 53.75) (width 0.25) (layer B.Cu) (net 2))
 (segment (start 110.1125 53.75) (end 109.4749 53.75) (width 0.25) (layer B.Cu) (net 2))
 (segment (start 110.75 53.75) (end 110.1125 53.75) (width 0.25) (layer B.Cu) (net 2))
 (segment (start 118.095 65.0251) (end 117.4516 65.0251) (width 0.25) (layer F.Cu) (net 2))
 (segment (start 117.4516 65.0251) (end 117.268 64.8415) (width 0.25) (layer F.Cu) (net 2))
 (segment (start 102.71 64.92) (end 103.8987 64.92) (width 0.25) (layer B.Cu) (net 2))
 (segment (start 118.095 63.85) (end 118.095 65.0251) (width 0.25) (layer F.Cu) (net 2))
 (segment (start 109 69.5) (end 115 69.5) (width 0.25) (layer B.Cu) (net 2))
 (segment (start 120.25 75.5) (end 119.4249 75.5) (width 0.25) (layer F.Cu) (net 2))
 (segment (start 115 69.5) (end 115 70.25) (width 0.25) (layer F.Cu) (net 2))
 (segment (start 115 70.25) (end 119.4249 74.6749) (width 0.25) (layer F.Cu) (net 2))
 (segment (start 119.4249 74.6749) (end 119.4249 75.5) (width 0.25) (layer F.Cu) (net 2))
 (via (at 117.268 64.8415) (size 0.6) (layers F.Cu B.Cu) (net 2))
 (segment (start 105.25 70) (end 107 68.25) (width 0.25) (layer F.Cu) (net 3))
 (segment (start 107 68.25) (end 118 68.25) (width 0.25) (layer F.Cu) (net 3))
 (segment (start 118 68.25) (end 119.365 69.615) (width 0.25) (layer F.Cu) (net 3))
 (segment (start 119.365 69.615) (end 119.365 71.15) (width 0.25) (layer F.Cu) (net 3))
 (segment (start 102.71 67.46) (end 104 68.75) (width 0.25) (layer B.Cu) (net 5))
 (segment (start 104 68.75) (end 106.5 68.75) (width 0.25) (layer B.Cu) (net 5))
 (segment (start 106.5 68.75) (end 107 68.25) (width 0.25) (layer B.Cu) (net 5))
 (segment (start 107 68.25) (end 116.75 68.25) (width 0.25) (layer B.Cu) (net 5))
 (segment (start 116.75 68.25) (end 118 69.5) (width 0.25) (layer B.Cu) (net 5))
 (segment (start 118 69.5) (end 118.095 69.595) (width 0.25) (layer F.Cu) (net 5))
 (segment (start 118.095 69.595) (end 118.095 71.15) (width 0.25) (layer F.Cu) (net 5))
 (via (at 118 69.5) (size 0.6) (layers F.Cu B.Cu) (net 5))
 (segment (start 121.905 63.85) (end 121.905 62.595) (width 0.25) (layer F.Cu) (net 6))
 (segment (start 121.905 62.595) (end 122 62.5) (width 0.25) (layer F.Cu) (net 6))
 (segment (start 122 62.5) (end 122 61.5) (width 0.25) (layer F.Cu) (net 6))
 (segment (start 105.25 64.92) (end 107.08 66.75) (width 0.25) (layer F.Cu) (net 6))
 (segment (start 107.08 66.75) (end 120 66.75) (width 0.25) (layer F.Cu) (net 6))
 (segment (start 120 66.75) (end 120.5 66.25) (width 0.25) (layer F.Cu) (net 6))
 (segment (start 120.5 66.25) (end 121.25 66.25) (width 0.25) (layer F.Cu) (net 6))
 (segment (start 121.25 66.25) (end 121.905 65.595) (width 0.25) (layer F.Cu) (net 6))
 (segment (start 121.905 65.595) (end 121.905 63.85) (width 0.25) (layer F.Cu) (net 6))
 (segment (start 119.5 58.25) (end 119.5 54.29) (width 0.25) (layer F.Cu) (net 7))
 (segment (start 119.5 54.29) (end 120.04 53.75) (width 0.25) (layer F.Cu) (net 7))
 (segment (start 106.5 58.25) (end 106.5 54.29) (width 0.25) (layer F.Cu) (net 8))
 (segment (start 106.5 54.29) (end 107.04 53.75) (width 0.25) (layer F.Cu) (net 8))
 (segment (start 112.75 58.25) (end 112.75 54.29) (width 0.25) (layer F.Cu) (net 9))
 (segment (start 112.75 54.29) (end 113.29 53.75) (width 0.25) (layer F.Cu) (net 9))
 (segment (start 120.635 63.85) (end 120.635 62.865) (width 0.25) (layer F.Cu) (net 10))
 (segment (start 120.635 62.865) (end 121.25 62.25) (width 0.25) (layer F.Cu) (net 10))
 (segment (start 121.25 62.25) (end 121.25 59.75) (width 0.25) (layer F.Cu) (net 10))
 (segment (start 121.25 59.75) (end 120.75 59.25) (width 0.25) (layer F.Cu) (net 10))
 (segment (start 120.75 59.25) (end 111.5 59.25) (width 0.25) (layer F.Cu) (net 10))
 (segment (start 111.5 59.25) (end 111.25 59) (width 0.25) (layer F.Cu) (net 10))
 (segment (start 111.25 59) (end 111.25 58.25) (width 0.25) (layer F.Cu) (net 10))
 (segment (start 112.75 65.5) (end 109 65.5) (width 0.25) (layer F.Cu) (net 11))
 (segment (start 115 65.5) (end 112.75 65.5) (width 0.25) (layer F.Cu) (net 11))
 (segment (start 115 65.5) (end 118.75 65.5) (width 0.25) (layer F.Cu) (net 11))
 (segment (start 118.75 65.5) (end 119.365 64.885) (width 0.25) (layer F.Cu) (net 11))
 (segment (start 119.365 64.885) (end 119.365 63.85) (width 0.25) (layer F.Cu) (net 11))
 (segment (start 112.75 63) (end 112.75 65.5) (width 0.25) (layer F.Cu) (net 11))
 (segment (start 117 58.25) (end 104 58.25) (width 0.25) (layer B.Cu) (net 4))
 (segment (start 104 58.25) (end 105 58.25) (width 0.25) (layer F.Cu) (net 4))
 (segment (start 118 58.25) (end 117 58.25) (width 0.25) (layer F.Cu) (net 4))
 (segment (start 120.635 71.15) (end 120.635 67.5) (width 0.25) (layer F.Cu) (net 4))
 (segment (start 120.635 67.5) (end 105.29 67.5) (width 0.25) (layer F.Cu) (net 4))
 (segment (start 105.29 67.5) (end 105.25 67.46) (width 0.25) (layer F.Cu) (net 4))
 (segment (start 117 58.25) (end 119.25 58.25) (width 0.25) (layer B.Cu) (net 4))
 (segment (start 119.25 58.25) (end 120.75 59.75) (width 0.25) (layer B.Cu) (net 4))
 (segment (start 120.75 59.75) (end 120.75 67.25) (width 0.25) (layer B.Cu) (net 4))
 (segment (start 120.75 67.25) (end 120.635 67.365) (width 0.25) (layer F.Cu) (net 4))
 (segment (start 120.635 67.365) (end 120.635 67.5) (width 0.25) (layer F.Cu) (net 4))
 (via (at 117 58.25) (size 0.6) (layers F.Cu B.Cu) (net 4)) (via (at 104 58.25) (size 0.6) (layers F.Cu B.Cu) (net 4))
 (via (at 120.75 67.25) (size 0.6) (layers F.Cu B.Cu) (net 4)))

